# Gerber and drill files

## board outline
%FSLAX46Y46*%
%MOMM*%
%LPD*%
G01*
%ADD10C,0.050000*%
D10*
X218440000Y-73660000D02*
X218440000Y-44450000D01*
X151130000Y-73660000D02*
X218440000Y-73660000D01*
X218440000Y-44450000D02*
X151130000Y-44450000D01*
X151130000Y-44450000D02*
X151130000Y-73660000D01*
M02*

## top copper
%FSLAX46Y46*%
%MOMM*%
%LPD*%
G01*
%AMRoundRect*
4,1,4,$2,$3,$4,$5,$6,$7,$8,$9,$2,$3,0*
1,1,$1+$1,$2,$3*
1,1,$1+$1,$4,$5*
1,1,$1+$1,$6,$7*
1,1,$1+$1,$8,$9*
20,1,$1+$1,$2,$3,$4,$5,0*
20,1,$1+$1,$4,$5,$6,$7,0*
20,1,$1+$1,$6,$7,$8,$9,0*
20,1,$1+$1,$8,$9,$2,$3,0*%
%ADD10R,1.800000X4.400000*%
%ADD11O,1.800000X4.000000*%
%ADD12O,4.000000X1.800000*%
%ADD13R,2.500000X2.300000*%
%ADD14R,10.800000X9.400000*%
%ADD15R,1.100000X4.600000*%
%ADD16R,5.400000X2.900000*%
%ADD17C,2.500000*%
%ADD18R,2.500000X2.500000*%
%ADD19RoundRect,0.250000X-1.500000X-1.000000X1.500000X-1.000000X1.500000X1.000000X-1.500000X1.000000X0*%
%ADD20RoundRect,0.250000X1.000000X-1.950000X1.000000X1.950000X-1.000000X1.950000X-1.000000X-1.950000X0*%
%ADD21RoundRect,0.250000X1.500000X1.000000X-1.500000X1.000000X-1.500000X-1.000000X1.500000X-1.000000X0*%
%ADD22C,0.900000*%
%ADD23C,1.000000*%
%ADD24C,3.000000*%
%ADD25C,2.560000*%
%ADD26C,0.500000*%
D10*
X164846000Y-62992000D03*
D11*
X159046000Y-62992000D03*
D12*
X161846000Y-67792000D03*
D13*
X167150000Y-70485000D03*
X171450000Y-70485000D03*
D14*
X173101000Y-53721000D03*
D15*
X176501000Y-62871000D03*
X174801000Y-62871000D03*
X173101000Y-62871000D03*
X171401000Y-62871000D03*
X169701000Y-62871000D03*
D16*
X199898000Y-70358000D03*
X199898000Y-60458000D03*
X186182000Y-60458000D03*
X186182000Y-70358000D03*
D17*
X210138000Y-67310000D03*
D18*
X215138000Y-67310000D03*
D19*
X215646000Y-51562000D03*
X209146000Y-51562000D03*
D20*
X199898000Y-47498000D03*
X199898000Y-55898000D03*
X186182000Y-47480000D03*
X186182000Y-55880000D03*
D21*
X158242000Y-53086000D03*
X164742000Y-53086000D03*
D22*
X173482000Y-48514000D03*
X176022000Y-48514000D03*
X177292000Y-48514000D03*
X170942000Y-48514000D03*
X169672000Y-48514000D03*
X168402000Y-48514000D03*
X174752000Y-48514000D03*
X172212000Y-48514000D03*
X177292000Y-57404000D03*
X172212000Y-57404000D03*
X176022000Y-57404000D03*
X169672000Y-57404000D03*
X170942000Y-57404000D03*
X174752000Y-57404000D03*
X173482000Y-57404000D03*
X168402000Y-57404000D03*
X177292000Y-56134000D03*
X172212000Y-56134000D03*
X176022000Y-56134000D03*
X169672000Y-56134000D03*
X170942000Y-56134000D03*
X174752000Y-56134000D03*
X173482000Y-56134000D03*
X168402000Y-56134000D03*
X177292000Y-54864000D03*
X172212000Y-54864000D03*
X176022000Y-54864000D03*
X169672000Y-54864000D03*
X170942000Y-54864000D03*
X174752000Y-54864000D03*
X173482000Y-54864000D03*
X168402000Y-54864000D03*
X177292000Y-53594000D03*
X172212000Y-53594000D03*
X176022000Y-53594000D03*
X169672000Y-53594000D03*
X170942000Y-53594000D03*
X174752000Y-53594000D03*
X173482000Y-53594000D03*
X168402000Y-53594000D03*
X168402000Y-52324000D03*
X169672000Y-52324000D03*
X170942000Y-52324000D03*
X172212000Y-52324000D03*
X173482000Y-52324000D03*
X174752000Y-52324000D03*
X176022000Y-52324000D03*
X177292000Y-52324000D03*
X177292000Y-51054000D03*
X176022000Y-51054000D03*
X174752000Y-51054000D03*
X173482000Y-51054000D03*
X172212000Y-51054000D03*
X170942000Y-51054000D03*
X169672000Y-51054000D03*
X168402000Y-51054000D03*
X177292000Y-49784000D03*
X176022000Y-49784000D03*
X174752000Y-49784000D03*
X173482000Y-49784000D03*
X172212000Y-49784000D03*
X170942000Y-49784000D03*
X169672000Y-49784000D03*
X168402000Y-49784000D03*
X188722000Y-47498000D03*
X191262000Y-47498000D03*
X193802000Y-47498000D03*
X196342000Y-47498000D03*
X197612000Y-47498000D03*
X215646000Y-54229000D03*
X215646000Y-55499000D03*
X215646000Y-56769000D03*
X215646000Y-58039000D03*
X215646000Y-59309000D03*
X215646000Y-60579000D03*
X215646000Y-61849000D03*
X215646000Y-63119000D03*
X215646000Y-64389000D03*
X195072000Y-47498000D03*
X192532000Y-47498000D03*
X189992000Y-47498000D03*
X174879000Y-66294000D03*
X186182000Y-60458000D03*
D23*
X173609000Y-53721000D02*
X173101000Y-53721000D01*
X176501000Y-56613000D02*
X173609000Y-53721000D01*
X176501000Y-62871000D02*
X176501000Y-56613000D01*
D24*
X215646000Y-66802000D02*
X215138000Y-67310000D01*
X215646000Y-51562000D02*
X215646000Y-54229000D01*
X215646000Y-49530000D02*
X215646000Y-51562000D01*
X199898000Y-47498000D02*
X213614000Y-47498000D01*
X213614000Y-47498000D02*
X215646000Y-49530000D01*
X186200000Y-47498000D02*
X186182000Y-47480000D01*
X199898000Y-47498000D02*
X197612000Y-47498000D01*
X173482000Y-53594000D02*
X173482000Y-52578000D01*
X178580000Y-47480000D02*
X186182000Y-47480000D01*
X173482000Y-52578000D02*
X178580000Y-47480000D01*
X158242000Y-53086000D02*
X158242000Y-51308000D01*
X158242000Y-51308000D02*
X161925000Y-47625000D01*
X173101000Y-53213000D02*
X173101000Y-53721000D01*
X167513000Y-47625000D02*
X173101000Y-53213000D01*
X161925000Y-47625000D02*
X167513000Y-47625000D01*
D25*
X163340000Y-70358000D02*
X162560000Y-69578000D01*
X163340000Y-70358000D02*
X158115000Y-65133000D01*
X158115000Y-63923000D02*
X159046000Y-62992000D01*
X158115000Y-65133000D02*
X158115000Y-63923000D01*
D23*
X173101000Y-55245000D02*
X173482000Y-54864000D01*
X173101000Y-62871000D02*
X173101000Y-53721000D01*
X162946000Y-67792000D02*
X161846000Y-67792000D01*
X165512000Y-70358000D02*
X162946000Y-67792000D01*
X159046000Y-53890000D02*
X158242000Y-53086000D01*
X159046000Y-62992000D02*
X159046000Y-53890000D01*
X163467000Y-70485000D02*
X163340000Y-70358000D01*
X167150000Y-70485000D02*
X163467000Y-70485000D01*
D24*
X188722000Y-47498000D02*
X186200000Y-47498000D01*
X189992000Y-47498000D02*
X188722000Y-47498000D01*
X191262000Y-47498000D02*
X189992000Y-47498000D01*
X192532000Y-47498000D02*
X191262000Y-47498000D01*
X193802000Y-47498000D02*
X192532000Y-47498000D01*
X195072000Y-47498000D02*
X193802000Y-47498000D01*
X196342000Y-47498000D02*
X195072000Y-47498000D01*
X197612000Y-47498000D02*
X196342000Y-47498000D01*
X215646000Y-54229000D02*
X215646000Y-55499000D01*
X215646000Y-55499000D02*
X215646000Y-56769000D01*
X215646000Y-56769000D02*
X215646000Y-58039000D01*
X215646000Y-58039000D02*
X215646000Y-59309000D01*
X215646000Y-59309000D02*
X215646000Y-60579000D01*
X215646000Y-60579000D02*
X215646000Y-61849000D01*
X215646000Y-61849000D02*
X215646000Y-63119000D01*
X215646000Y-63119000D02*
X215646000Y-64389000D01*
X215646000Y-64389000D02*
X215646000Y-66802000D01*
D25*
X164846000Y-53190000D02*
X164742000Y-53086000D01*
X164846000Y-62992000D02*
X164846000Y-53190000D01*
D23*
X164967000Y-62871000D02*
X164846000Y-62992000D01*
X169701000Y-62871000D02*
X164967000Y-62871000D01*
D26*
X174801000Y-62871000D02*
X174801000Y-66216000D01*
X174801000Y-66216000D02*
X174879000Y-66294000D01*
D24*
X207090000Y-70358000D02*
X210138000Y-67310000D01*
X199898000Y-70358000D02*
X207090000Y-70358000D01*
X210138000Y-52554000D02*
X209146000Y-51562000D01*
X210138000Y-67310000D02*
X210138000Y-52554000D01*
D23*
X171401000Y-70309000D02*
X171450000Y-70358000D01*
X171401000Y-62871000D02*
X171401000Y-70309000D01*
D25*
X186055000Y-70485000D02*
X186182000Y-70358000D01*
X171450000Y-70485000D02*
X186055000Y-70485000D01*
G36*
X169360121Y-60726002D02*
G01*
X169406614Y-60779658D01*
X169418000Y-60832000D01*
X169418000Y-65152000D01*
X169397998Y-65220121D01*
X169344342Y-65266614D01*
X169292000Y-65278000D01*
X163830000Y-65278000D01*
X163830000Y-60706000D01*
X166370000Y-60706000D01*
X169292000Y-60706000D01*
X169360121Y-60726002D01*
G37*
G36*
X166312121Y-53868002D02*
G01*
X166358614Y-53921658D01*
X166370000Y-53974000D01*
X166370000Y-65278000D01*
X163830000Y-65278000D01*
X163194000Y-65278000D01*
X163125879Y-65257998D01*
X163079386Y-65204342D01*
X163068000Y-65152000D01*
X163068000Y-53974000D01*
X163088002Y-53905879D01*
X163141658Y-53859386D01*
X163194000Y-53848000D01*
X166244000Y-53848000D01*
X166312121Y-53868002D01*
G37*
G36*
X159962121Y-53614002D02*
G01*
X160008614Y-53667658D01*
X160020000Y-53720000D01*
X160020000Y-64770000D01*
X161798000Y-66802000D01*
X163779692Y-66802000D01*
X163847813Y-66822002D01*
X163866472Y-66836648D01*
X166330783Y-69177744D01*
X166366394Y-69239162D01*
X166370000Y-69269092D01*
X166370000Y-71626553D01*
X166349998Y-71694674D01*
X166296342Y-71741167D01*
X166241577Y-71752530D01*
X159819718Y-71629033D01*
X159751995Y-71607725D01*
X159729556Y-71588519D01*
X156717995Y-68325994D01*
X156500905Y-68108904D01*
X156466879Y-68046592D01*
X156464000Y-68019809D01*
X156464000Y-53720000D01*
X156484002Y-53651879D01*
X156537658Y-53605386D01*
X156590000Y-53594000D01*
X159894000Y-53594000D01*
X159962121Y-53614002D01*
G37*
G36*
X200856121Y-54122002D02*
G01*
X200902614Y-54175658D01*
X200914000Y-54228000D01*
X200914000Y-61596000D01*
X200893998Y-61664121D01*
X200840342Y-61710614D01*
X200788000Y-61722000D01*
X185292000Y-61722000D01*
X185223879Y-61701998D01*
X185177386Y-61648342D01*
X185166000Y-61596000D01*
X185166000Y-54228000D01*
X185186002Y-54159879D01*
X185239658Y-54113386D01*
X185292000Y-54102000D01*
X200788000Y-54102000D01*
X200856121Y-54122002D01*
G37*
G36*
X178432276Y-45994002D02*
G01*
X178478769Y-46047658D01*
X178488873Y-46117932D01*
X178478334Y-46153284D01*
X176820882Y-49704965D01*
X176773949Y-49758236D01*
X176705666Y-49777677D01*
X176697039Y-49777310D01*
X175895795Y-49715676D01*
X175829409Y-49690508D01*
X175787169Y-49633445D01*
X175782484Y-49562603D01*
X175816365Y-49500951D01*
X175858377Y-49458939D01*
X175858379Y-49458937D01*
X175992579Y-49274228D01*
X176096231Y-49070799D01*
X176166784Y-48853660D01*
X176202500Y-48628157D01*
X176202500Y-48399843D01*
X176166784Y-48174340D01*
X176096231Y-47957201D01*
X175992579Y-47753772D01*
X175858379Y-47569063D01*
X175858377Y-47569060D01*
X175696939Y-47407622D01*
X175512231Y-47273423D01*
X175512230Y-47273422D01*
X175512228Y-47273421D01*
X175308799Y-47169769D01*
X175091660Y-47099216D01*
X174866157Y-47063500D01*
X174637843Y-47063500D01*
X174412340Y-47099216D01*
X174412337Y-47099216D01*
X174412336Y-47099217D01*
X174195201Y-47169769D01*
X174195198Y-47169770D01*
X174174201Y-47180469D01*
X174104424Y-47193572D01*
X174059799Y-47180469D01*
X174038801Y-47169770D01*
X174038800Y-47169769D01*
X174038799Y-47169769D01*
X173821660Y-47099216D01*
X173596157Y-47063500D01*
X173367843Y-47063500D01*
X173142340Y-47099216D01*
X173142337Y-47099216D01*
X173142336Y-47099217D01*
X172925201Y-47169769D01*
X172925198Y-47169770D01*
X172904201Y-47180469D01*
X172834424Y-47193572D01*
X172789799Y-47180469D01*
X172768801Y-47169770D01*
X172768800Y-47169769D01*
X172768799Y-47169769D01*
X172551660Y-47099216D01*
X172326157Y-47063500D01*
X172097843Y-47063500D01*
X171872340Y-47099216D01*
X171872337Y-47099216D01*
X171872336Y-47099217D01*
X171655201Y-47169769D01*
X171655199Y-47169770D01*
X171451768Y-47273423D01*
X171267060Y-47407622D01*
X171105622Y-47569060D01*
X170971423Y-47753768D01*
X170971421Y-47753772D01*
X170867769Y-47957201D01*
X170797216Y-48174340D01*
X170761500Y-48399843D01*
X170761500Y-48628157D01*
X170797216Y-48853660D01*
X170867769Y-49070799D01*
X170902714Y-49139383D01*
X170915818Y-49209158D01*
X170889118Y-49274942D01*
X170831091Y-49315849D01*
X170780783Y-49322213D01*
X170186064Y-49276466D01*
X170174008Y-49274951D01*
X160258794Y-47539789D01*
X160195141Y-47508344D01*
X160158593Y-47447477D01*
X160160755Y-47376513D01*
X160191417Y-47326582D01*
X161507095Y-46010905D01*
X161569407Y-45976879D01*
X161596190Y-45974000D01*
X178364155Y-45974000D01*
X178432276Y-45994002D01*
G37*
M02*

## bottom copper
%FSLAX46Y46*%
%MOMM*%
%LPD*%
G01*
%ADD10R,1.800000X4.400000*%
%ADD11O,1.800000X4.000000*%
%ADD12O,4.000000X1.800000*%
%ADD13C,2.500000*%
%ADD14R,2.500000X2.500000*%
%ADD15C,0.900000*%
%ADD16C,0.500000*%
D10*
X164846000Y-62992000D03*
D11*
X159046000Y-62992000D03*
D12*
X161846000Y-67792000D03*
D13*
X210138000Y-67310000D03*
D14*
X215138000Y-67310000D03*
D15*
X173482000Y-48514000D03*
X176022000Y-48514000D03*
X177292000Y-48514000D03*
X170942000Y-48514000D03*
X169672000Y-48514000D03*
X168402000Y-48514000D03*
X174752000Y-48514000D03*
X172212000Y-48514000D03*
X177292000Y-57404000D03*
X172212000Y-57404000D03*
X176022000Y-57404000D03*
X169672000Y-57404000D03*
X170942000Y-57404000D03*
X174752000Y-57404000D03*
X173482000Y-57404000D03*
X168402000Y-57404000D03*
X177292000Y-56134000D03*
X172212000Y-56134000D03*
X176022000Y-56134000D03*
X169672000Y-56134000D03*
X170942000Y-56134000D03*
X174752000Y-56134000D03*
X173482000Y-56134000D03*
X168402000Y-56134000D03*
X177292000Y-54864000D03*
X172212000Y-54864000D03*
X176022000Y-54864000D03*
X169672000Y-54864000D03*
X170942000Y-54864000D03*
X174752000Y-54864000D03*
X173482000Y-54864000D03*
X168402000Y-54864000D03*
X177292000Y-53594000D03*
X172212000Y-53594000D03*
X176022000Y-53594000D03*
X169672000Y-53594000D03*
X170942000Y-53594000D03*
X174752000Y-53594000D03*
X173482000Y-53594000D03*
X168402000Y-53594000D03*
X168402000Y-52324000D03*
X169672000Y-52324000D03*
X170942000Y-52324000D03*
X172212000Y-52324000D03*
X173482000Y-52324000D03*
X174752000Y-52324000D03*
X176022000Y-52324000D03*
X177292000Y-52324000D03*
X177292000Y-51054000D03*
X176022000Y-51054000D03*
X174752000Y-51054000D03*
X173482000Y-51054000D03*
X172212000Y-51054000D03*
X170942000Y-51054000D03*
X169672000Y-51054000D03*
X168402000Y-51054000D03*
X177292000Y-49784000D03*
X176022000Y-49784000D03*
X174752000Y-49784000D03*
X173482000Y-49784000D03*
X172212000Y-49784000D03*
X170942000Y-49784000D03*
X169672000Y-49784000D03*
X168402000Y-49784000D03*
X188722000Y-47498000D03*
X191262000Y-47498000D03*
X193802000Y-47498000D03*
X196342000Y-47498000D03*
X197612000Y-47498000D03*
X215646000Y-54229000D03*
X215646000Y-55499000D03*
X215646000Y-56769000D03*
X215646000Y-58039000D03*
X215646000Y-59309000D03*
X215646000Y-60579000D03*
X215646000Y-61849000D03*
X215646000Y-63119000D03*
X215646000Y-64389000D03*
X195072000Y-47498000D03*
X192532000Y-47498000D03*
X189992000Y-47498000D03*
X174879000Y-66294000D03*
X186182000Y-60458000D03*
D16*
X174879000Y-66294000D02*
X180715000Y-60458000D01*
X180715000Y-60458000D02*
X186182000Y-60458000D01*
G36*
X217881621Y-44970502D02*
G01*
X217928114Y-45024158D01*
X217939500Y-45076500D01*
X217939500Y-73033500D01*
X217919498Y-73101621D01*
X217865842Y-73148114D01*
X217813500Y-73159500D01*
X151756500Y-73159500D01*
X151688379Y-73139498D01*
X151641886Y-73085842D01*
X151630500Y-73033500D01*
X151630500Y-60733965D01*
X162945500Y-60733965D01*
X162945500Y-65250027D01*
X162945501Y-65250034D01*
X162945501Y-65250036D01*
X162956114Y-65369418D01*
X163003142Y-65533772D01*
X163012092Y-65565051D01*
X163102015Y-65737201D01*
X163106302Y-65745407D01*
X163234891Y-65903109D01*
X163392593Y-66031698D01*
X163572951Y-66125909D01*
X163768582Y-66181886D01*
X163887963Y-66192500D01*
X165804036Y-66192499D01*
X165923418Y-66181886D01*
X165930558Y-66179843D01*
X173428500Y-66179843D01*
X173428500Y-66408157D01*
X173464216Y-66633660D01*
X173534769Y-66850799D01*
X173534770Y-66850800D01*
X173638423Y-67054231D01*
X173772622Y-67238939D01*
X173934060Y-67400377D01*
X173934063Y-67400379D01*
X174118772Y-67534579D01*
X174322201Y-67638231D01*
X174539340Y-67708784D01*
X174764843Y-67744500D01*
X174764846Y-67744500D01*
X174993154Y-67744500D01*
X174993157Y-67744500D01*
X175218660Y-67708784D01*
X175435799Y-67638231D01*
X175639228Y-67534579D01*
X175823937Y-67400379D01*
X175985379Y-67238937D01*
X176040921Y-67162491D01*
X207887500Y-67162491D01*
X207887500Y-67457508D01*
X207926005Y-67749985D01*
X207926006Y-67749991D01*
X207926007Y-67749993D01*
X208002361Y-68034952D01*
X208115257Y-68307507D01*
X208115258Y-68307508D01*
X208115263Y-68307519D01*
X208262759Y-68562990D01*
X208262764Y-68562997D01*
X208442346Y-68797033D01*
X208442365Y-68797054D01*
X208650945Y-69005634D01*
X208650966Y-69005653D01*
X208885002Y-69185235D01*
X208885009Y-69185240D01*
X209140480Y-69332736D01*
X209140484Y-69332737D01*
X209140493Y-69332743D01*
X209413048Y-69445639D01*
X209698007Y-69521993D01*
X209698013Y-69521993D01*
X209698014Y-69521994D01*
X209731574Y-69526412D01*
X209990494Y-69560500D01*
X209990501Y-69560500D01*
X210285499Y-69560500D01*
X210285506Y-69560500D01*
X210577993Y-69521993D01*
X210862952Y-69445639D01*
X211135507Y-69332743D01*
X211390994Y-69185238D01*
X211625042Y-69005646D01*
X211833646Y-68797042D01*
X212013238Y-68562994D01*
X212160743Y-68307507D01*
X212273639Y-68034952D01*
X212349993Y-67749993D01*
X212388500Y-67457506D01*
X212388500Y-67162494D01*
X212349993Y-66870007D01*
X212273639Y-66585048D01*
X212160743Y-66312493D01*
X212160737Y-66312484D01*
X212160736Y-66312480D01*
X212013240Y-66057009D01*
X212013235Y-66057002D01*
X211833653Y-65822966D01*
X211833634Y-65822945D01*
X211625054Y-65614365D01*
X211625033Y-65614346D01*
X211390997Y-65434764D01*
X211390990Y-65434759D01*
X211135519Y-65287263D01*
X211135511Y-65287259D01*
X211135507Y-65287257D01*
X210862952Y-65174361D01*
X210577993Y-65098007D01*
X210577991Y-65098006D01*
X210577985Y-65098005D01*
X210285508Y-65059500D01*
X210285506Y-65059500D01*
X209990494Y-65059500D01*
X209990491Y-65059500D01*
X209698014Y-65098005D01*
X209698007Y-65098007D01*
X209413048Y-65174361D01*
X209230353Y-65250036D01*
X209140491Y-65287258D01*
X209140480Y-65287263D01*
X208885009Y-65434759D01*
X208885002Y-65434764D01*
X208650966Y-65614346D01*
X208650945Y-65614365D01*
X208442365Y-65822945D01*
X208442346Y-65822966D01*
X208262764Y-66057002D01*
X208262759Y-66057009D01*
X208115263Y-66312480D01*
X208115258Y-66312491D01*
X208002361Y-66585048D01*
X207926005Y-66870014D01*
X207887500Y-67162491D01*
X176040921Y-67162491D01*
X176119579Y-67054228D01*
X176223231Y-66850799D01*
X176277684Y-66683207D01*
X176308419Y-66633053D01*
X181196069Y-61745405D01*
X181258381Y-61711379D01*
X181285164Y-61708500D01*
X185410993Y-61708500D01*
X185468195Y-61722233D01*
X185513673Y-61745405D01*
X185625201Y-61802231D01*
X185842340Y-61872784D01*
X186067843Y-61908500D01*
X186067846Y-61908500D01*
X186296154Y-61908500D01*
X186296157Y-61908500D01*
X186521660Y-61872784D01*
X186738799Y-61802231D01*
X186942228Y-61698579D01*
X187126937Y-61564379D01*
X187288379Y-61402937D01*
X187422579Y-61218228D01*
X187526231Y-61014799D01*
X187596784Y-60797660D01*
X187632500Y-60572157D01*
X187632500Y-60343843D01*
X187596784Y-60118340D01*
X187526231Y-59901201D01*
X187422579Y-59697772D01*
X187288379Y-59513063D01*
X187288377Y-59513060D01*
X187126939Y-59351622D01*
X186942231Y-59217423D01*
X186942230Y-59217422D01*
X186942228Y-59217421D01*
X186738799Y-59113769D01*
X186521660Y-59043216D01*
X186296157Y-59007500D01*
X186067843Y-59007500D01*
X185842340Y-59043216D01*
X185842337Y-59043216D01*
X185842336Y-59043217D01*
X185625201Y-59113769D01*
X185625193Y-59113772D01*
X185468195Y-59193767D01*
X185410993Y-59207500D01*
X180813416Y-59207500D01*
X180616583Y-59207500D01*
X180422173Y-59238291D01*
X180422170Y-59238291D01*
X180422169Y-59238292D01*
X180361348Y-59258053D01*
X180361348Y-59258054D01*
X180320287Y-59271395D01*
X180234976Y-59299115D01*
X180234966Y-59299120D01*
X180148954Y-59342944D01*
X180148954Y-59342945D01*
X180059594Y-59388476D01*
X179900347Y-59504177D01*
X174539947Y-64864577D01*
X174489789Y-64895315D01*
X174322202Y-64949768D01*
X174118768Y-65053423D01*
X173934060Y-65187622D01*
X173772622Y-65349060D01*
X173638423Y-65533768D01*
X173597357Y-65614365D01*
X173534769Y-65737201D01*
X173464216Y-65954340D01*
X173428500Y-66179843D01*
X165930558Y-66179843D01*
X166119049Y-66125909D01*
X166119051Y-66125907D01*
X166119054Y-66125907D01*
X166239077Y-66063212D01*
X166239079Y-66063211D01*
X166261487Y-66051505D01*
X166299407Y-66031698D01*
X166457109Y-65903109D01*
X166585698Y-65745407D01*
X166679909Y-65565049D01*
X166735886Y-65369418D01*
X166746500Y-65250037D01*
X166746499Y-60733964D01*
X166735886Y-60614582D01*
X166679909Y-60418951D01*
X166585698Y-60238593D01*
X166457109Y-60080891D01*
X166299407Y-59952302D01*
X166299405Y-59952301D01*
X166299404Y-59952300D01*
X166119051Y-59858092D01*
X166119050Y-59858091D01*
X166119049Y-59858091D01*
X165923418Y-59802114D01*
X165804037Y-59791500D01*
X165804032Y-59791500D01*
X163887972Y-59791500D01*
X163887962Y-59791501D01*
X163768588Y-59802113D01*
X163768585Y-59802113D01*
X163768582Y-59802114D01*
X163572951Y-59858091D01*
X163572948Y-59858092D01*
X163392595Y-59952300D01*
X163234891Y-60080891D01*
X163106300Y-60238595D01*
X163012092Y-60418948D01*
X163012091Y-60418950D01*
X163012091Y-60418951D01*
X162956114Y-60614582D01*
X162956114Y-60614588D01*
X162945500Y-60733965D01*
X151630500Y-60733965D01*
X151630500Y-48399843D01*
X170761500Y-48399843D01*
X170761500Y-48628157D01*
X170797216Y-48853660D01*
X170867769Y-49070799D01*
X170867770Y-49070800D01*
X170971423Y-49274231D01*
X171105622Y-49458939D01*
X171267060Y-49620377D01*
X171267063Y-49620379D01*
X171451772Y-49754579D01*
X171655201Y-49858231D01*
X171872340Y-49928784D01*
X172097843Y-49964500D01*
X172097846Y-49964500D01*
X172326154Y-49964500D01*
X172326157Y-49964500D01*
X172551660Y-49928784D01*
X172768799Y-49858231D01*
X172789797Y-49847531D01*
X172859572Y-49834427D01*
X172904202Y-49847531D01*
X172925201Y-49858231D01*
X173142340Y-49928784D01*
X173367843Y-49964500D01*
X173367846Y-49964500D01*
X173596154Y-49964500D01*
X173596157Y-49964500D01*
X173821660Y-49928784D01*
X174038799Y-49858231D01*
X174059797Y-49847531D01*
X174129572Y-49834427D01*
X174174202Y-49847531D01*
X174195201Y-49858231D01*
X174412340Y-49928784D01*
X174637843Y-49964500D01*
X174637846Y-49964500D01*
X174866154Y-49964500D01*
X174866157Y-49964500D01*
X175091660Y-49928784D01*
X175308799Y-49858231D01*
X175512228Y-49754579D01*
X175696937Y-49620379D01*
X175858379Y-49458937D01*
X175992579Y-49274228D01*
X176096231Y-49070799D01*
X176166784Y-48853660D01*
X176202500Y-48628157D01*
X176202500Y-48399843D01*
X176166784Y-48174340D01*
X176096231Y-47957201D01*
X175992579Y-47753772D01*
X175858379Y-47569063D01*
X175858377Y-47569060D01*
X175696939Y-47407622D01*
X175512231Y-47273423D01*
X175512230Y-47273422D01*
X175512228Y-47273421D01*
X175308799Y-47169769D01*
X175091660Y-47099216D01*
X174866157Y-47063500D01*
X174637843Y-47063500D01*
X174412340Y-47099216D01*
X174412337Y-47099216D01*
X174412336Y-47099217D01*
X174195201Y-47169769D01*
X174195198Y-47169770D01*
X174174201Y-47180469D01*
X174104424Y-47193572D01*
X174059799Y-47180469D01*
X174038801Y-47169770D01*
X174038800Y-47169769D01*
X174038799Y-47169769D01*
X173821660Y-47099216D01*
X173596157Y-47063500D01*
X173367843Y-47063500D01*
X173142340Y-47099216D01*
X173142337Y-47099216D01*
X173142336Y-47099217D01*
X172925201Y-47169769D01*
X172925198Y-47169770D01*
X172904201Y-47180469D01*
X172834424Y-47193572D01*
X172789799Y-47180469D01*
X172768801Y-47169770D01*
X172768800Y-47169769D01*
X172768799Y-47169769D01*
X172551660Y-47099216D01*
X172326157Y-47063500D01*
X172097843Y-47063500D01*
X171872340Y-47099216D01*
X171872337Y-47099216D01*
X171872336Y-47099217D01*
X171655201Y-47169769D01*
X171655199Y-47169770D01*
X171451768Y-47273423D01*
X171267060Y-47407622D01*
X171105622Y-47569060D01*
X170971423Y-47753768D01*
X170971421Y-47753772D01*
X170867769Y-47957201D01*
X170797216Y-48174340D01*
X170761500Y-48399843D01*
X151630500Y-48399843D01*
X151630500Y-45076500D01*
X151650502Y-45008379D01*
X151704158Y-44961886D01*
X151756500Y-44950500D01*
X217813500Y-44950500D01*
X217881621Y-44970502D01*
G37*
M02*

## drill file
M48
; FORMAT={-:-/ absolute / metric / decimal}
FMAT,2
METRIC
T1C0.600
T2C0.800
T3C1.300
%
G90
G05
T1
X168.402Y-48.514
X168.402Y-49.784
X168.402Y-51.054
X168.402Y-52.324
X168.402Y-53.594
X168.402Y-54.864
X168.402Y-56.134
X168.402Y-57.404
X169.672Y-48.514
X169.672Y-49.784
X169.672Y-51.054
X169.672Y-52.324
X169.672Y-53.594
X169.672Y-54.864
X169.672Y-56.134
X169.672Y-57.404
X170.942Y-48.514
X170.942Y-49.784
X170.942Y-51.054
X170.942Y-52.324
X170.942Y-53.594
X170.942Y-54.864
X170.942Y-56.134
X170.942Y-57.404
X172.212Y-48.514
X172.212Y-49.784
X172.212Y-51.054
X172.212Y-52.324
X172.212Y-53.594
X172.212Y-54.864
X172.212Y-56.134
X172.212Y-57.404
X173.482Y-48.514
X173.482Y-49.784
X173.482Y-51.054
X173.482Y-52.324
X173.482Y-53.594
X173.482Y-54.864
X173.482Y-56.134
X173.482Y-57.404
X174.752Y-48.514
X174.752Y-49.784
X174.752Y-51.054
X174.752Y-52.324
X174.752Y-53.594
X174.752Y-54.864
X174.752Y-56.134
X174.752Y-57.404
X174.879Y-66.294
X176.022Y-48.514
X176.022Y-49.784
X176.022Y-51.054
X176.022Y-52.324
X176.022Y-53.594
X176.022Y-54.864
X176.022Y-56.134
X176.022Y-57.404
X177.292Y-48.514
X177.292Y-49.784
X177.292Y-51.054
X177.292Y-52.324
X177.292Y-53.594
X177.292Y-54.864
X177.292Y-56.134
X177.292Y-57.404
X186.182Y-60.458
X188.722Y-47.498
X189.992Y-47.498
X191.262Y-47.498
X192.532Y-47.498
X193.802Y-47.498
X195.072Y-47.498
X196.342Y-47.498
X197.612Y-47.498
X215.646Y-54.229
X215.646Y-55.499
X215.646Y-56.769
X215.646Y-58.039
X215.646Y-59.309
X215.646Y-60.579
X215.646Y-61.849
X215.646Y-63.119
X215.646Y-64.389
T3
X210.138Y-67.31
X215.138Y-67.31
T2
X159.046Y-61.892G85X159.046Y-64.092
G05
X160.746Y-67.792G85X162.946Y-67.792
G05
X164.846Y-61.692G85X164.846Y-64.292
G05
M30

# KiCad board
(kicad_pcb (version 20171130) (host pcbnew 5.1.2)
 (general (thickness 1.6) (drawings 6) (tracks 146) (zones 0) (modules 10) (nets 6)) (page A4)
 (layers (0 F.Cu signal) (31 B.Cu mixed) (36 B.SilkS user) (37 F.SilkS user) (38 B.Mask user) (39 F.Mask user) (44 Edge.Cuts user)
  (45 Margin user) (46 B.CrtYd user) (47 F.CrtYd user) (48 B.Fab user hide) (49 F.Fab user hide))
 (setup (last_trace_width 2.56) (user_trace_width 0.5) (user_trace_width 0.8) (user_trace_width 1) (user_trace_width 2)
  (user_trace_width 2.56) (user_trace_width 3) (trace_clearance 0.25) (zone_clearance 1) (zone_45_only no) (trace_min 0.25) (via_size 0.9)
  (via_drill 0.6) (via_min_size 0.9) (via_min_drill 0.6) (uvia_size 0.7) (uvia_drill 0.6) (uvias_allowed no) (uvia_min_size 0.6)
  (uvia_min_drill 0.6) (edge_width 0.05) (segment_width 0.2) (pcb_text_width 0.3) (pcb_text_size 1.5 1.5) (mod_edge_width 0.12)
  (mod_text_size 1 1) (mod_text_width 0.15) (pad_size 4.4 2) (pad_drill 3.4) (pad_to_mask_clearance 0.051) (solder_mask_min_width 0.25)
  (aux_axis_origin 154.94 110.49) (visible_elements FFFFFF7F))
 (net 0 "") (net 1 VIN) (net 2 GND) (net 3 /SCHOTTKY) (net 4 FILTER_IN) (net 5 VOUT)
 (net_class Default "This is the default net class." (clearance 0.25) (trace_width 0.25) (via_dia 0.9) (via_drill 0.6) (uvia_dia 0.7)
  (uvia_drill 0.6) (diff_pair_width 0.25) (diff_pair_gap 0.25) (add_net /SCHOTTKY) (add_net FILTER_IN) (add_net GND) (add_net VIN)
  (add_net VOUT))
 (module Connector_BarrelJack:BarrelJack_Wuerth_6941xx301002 (layer F.Cu) (at 164.846 62.992 270)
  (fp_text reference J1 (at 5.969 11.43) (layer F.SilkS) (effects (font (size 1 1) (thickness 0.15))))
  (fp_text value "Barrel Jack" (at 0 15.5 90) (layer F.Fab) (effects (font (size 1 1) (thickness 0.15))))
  (pad 1 thru_hole rect (at 0 0 270) (size 4.4 1.8) (drill oval 3.4 0.8) (layers *.Cu *.Mask) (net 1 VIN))
  (pad 2 thru_hole oval (at 0 5.8 270) (size 4 1.8) (drill oval 3 0.8) (layers *.Cu *.Mask) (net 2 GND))
  (pad 3 thru_hole oval (at 4.8 3) (size 4 1.8) (drill oval 3 0.8) (layers *.Cu *.Mask) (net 2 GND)))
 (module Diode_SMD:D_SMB (layer F.Cu) (at 169.3 70.485 180)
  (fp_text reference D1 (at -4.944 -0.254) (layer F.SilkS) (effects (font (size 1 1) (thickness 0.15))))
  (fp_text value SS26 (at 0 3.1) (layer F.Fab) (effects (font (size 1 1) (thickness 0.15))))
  (pad 2 smd rect (at 2.15 0 180) (size 2.5 2.3) (layers F.Cu F.Paste F.Mask) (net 2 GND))
  (pad 1 smd rect (at -2.15 0 180) (size 2.5 2.3) (layers F.Cu F.Paste F.Mask) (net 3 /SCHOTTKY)))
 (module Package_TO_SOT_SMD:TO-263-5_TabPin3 (layer F.Cu) (at 173.101 57.096 90)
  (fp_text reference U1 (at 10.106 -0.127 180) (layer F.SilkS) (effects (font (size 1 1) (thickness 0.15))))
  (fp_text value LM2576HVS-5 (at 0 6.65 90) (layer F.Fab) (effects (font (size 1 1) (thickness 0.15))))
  (pad "" smd rect (at 0.95 2.775 90) (size 4.55 5.25) (layers F.Paste))
  (pad "" smd rect (at 5.8 -2.775 90) (size 4.55 5.25) (layers F.Paste))
  (pad "" smd rect (at 0.95 -2.775 90) (size 4.55 5.25) (layers F.Paste))
  (pad "" smd rect (at 5.8 2.775 90) (size 4.55 5.25) (layers F.Paste))
  (pad 3 smd rect (at 3.375 0 90) (size 9.4 10.8) (layers F.Cu F.Mask) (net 2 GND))
  (pad 5 smd rect (at -5.775 3.4 90) (size 4.6 1.1) (layers F.Cu F.Paste F.Mask) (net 2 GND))
  (pad 4 smd rect (at -5.775 1.7 90) (size 4.6 1.1) (layers F.Cu F.Paste F.Mask) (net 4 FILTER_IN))
  (pad 3 smd rect (at -5.775 0 90) (size 4.6 1.1) (layers F.Cu F.Paste F.Mask) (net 2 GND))
  (pad 2 smd rect (at -5.775 -1.7 90) (size 4.6 1.1) (layers F.Cu F.Paste F.Mask) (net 3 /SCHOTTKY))
  (pad 1 smd rect (at -5.775 -3.4 90) (size 4.6 1.1) (layers F.Cu F.Paste F.Mask) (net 1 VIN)))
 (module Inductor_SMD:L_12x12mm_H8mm (layer F.Cu) (at 199.898 65.408 270)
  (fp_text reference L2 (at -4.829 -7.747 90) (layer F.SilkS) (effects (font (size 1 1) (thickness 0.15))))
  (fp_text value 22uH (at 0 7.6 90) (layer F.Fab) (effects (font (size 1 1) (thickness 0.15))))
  (pad 2 smd rect (at 4.95 0 270) (size 2.9 5.4) (layers F.Cu F.Paste F.Mask) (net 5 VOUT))
  (pad 1 smd rect (at -4.95 0 270) (size 2.9 5.4) (layers F.Cu F.Paste F.Mask) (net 4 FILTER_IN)))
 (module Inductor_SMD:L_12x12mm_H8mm (layer F.Cu) (at 186.182 65.408 90)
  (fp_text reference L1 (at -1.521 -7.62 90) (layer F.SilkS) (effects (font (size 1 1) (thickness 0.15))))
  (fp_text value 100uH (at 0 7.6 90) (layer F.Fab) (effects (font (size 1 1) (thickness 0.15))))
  (pad 2 smd rect (at 4.95 0 90) (size 2.9 5.4) (layers F.Cu F.Paste F.Mask) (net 4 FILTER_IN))
  (pad 1 smd rect (at -4.95 0 90) (size 2.9 5.4) (layers F.Cu F.Paste F.Mask) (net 3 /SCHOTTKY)))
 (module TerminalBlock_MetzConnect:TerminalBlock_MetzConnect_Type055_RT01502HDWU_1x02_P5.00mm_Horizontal (layer F.Cu) (at 215.138 67.31 180)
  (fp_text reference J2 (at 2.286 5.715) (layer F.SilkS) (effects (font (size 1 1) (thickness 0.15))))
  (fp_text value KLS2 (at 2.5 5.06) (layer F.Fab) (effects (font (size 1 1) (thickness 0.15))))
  (pad 2 thru_hole circle (at 5 0 180) (size 2.5 2.5) (drill 1.3) (layers *.Cu *.Mask) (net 5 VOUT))
  (pad 1 thru_hole rect (at 0 0 180) (size 2.5 2.5) (drill 1.3) (layers *.Cu *.Mask) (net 2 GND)))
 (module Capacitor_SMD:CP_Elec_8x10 (layer F.Cu) (at 212.396 51.562)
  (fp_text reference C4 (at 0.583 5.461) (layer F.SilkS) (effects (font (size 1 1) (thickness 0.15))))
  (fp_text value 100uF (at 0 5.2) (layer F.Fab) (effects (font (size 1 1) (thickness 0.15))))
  (pad 2 smd roundrect (at 3.25 0) (size 3.5 2.5) (layers F.Cu F.Paste F.Mask) (roundrect_rratio 0.1) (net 2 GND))
  (pad 1 smd roundrect (at -3.25 0) (size 3.5 2.5) (layers F.Cu F.Paste F.Mask) (roundrect_rratio 0.1) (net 5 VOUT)))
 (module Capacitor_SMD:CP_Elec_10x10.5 (layer F.Cu) (at 199.898 51.698 90)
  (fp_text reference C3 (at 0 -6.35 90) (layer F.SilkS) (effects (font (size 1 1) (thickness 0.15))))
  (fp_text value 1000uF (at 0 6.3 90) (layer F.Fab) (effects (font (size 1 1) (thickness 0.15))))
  (pad 2 smd roundrect (at 4.2 0 90) (size 4.4 2.5) (layers F.Cu F.Paste F.Mask) (roundrect_rratio 0.1) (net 2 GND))
  (pad 1 smd roundrect (at -4.2 0 90) (size 4.4 2.5) (layers F.Cu F.Paste F.Mask) (roundrect_rratio 0.1) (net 4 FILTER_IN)))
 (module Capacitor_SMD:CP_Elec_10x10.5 (layer F.Cu) (at 186.182 51.68 90)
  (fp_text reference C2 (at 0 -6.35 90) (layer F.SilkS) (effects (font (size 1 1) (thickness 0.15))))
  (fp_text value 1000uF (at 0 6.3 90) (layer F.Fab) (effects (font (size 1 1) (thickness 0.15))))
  (pad 2 smd roundrect (at 4.2 0 90) (size 4.4 2.5) (layers F.Cu F.Paste F.Mask) (roundrect_rratio 0.1) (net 2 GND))
  (pad 1 smd roundrect (at -4.2 0 90) (size 4.4 2.5) (layers F.Cu F.Paste F.Mask) (roundrect_rratio 0.1) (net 4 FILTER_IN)))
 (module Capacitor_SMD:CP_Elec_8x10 (layer F.Cu) (at 161.492 53.086 180)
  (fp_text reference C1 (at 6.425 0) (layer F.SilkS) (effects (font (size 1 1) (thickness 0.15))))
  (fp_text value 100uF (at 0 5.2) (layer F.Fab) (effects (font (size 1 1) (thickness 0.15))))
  (pad 2 smd roundrect (at 3.25 0 180) (size 3.5 2.5) (layers F.Cu F.Paste F.Mask) (roundrect_rratio 0.1) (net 2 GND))
  (pad 1 smd roundrect (at -3.25 0 180) (size 3.5 2.5) (layers F.Cu F.Paste F.Mask) (roundrect_rratio 0.1) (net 1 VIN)))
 (gr_line (start 218.44 73.66) (end 218.44 44.45) (layer Edge.Cuts) (width 0.05))
 (gr_line (start 151.13 73.66) (end 218.44 73.66) (layer Edge.Cuts) (width 0.05))
 (gr_line (start 218.44 44.45) (end 151.13 44.45) (layer Edge.Cuts) (width 0.05))
 (gr_line (start 151.13 44.45) (end 151.13 73.66) (layer Edge.Cuts) (width 0.05))
 (via (at 173.482 48.514) (size 0.9) (drill 0.6) (layers F.Cu B.Cu) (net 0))
 (via (at 176.022 48.514) (size 0.9) (drill 0.6) (layers F.Cu B.Cu) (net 2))
 (via (at 177.292 48.514) (size 0.9) (drill 0.6) (layers F.Cu B.Cu) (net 2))
 (via (at 170.942 48.514) (size 0.9) (drill 0.6) (layers F.Cu B.Cu) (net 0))
 (via (at 169.672 48.514) (size 0.9) (drill 0.6) (layers F.Cu B.Cu) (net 2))
 (via (at 168.402 48.514) (size 0.9) (drill 0.6) (layers F.Cu B.Cu) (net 2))
 (via (at 174.752 48.514) (size 0.9) (drill 0.6) (layers F.Cu B.Cu) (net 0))
 (via (at 172.212 48.514) (size 0.9) (drill 0.6) (layers F.Cu B.Cu) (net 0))
 (via (at 177.292 57.404) (size 0.9) (drill 0.6) (layers F.Cu B.Cu) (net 2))
 (via (at 172.212 57.404) (size 0.9) (drill 0.6) (layers F.Cu B.Cu) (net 2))
 (via (at 176.022 57.404) (size 0.9) (drill 0.6) (layers F.Cu B.Cu) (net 2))
 (via (at 169.672 57.404) (size 0.9) (drill 0.6) (layers F.Cu B.Cu) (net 2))
 (via (at 170.942 57.404) (size 0.9) (drill 0.6) (layers F.Cu B.Cu) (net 2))
 (via (at 174.752 57.404) (size 0.9) (drill 0.6) (layers F.Cu B.Cu) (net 2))
 (via (at 173.482 57.404) (size 0.9) (drill 0.6) (layers F.Cu B.Cu) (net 2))
 (via (at 168.402 57.404) (size 0.9) (drill 0.6) (layers F.Cu B.Cu) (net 2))
 (via (at 177.292 56.134) (size 0.9) (drill 0.6) (layers F.Cu B.Cu) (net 2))
 (via (at 172.212 56.134) (size 0.9) (drill 0.6) (layers F.Cu B.Cu) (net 2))
 (via (at 176.022 56.134) (size 0.9) (drill 0.6) (layers F.Cu B.Cu) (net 2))
 (via (at 169.672 56.134) (size 0.9) (drill 0.6) (layers F.Cu B.Cu) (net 2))
 (via (at 170.942 56.134) (size 0.9) (drill 0.6) (layers F.Cu B.Cu) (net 2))
 (via (at 174.752 56.134) (size 0.9) (drill 0.6) (layers F.Cu B.Cu) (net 2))
 (via (at 173.482 56.134) (size 0.9) (drill 0.6) (layers F.Cu B.Cu) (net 2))
 (via (at 168.402 56.134) (size 0.9) (drill 0.6) (layers F.Cu B.Cu) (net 2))
 (via (at 177.292 54.864) (size 0.9) (drill 0.6) (layers F.Cu B.Cu) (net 2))
 (via (at 172.212 54.864) (size 0.9) (drill 0.6) (layers F.Cu B.Cu) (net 2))
 (via (at 176.022 54.864) (size 0.9) (drill 0.6) (layers F.Cu B.Cu) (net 2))
 (via (at 169.672 54.864) (size 0.9) (drill 0.6) (layers F.Cu B.Cu) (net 2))
 (via (at 170.942 54.864) (size 0.9) (drill 0.6) (layers F.Cu B.Cu) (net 2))
 (via (at 174.752 54.864) (size 0.9) (drill 0.6) (layers F.Cu B.Cu) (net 2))
 (via (at 173.482 54.864) (size 0.9) (drill 0.6) (layers F.Cu B.Cu) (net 2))
 (via (at 168.402 54.864) (size 0.9) (drill 0.6) (layers F.Cu B.Cu) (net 2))
 (via (at 177.292 53.594) (size 0.9) (drill 0.6) (layers F.Cu B.Cu) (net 2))
 (via (at 172.212 53.594) (size 0.9) (drill 0.6) (layers F.Cu B.Cu) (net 2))
 (via (at 176.022 53.594) (size 0.9) (drill 0.6) (layers F.Cu B.Cu) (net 2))
 (via (at 169.672 53.594) (size 0.9) (drill 0.6) (layers F.Cu B.Cu) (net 2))
 (via (at 170.942 53.594) (size 0.9) (drill 0.6) (layers F.Cu B.Cu) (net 2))
 (via (at 174.752 53.594) (size 0.9) (drill 0.6) (layers F.Cu B.Cu) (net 2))
 (via (at 173.482 53.594) (size 0.9) (drill 0.6) (layers F.Cu B.Cu) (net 2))
 (via (at 168.402 53.594) (size 0.9) (drill 0.6) (layers F.Cu B.Cu) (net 2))
 (via (at 168.402 52.324) (size 0.9) (drill 0.6) (layers F.Cu B.Cu) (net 2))
 (via (at 169.672 52.324) (size 0.9) (drill 0.6) (layers F.Cu B.Cu) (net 2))
 (via (at 170.942 52.324) (size 0.9) (drill 0.6) (layers F.Cu B.Cu) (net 2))
 (via (at 172.212 52.324) (size 0.9) (drill 0.6) (layers F.Cu B.Cu) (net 2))
 (via (at 173.482 52.324) (size 0.9) (drill 0.6) (layers F.Cu B.Cu) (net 2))
 (via (at 174.752 52.324) (size 0.9) (drill 0.6) (layers F.Cu B.Cu) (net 2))
 (via (at 176.022 52.324) (size 0.9) (drill 0.6) (layers F.Cu B.Cu) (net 2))
 (via (at 177.292 52.324) (size 0.9) (drill 0.6) (layers F.Cu B.Cu) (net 2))
 (via (at 177.292 51.054) (size 0.9) (drill 0.6) (layers F.Cu B.Cu) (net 2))
 (via (at 176.022 51.054) (size 0.9) (drill 0.6) (layers F.Cu B.Cu) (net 2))
 (via (at 174.752 51.054) (size 0.9) (drill 0.6) (layers F.Cu B.Cu) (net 2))
 (via (at 173.482 51.054) (size 0.9) (drill 0.6) (layers F.Cu B.Cu) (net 2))
 (via (at 172.212 51.054) (size 0.9) (drill 0.6) (layers F.Cu B.Cu) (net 2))
 (via (at 170.942 51.054) (size 0.9) (drill 0.6) (layers F.Cu B.Cu) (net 2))
 (via (at 169.672 51.054) (size 0.9) (drill 0.6) (layers F.Cu B.Cu) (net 2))
 (via (at 168.402 51.054) (size 0.9) (drill 0.6) (layers F.Cu B.Cu) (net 2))
 (via (at 177.292 49.784) (size 0.9) (drill 0.6) (layers F.Cu B.Cu) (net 2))
 (via (at 176.022 49.784) (size 0.9) (drill 0.6) (layers F.Cu B.Cu) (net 2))
 (via (at 174.752 49.784) (size 0.9) (drill 0.6) (layers F.Cu B.Cu) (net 2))
 (via (at 173.482 49.784) (size 0.9) (drill 0.6) (layers F.Cu B.Cu) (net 2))
 (via (at 172.212 49.784) (size 0.9) (drill 0.6) (layers F.Cu B.Cu) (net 2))
 (via (at 170.942 49.784) (size 0.9) (drill 0.6) (layers F.Cu B.Cu) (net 2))
 (via (at 169.672 49.784) (size 0.9) (drill 0.6) (layers F.Cu B.Cu) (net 2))
 (via (at 168.402 49.784) (size 0.9) (drill 0.6) (layers F.Cu B.Cu) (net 2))
 (segment (start 173.609 53.721) (end 173.101 53.721) (width 1) (layer F.Cu) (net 2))
 (segment (start 176.501 56.613) (end 173.609 53.721) (width 1) (layer F.Cu) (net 2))
 (segment (start 176.501 62.871) (end 176.501 56.613) (width 1) (layer F.Cu) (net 2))
 (segment (start 215.646 66.802) (end 215.138 67.31) (width 3) (layer F.Cu) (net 2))
 (segment (start 215.646 51.562) (end 215.646 54.229) (width 3) (layer F.Cu) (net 2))
 (segment (start 215.646 49.53) (end 215.646 51.562) (width 3) (layer F.Cu) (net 2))
 (segment (start 199.898 47.498) (end 213.614 47.498) (width 3) (layer F.Cu) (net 2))
 (segment (start 213.614 47.498) (end 215.646 49.53) (width 3) (layer F.Cu) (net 2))
 (segment (start 186.2 47.498) (end 186.182 47.48) (width 3) (layer F.Cu) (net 2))
 (segment (start 199.898 47.498) (end 197.612 47.498) (width 3) (layer F.Cu) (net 2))
 (segment (start 173.482 53.594) (end 173.482 52.578) (width 3) (layer F.Cu) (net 2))
 (segment (start 178.58 47.48) (end 186.182 47.48) (width 3) (layer F.Cu) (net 2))
 (segment (start 173.482 52.578) (end 178.58 47.48) (width 3) (layer F.Cu) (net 2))
 (segment (start 158.242 53.086) (end 158.242 51.308) (width 3) (layer F.Cu) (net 2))
 (segment (start 158.242 51.308) (end 161.925 47.625) (width 3) (layer F.Cu) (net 2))
 (segment (start 173.101 53.213) (end 173.101 53.721) (width 3) (layer F.Cu) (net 2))
 (segment (start 167.513 47.625) (end 173.101 53.213) (width 3) (layer F.Cu) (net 2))
 (segment (start 161.925 47.625) (end 167.513 47.625) (width 3) (layer F.Cu) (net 2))
 (segment (start 163.34 70.358) (end 162.56 69.578) (width 2.56) (layer F.Cu) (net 2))
 (segment (start 163.34 70.358) (end 158.115 65.133) (width 2.56) (layer F.Cu) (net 2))
 (segment (start 158.115 63.923) (end 159.046 62.992) (width 2.56) (layer F.Cu) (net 2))
 (segment (start 158.115 65.133) (end 158.115 63.923) (width 2.56) (layer F.Cu) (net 2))
 (segment (start 173.101 55.245) (end 173.482 54.864) (width 1) (layer F.Cu) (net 2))
 (segment (start 173.101 62.871) (end 173.101 53.721) (width 1) (layer F.Cu) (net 2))
 (segment (start 162.946 67.792) (end 161.846 67.792) (width 1) (layer F.Cu) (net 2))
 (segment (start 165.512 70.358) (end 162.946 67.792) (width 1) (layer F.Cu) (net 2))
 (segment (start 159.046 53.89) (end 158.242 53.086) (width 1) (layer F.Cu) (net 2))
 (segment (start 159.046 62.992) (end 159.046 53.89) (width 1) (layer F.Cu) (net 2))
 (segment (start 163.467 70.485) (end 163.34 70.358) (width 1) (layer F.Cu) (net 2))
 (segment (start 167.15 70.485) (end 163.467 70.485) (width 1) (layer F.Cu) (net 2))
 (segment (start 188.722 47.498) (end 186.2 47.498) (width 3) (layer F.Cu) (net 2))
 (via (at 188.722 47.498) (size 0.9) (drill 0.6) (layers F.Cu B.Cu) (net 2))
 (segment (start 189.992 47.498) (end 188.722 47.498) (width 3) (layer F.Cu) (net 2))
 (segment (start 191.262 47.498) (end 189.992 47.498) (width 3) (layer F.Cu) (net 2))
 (via (at 191.262 47.498) (size 0.9) (drill 0.6) (layers F.Cu B.Cu) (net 2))
 (segment (start 192.532 47.498) (end 191.262 47.498) (width 3) (layer F.Cu) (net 2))
 (segment (start 193.802 47.498) (end 192.532 47.498) (width 3) (layer F.Cu) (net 2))
 (via (at 193.802 47.498) (size 0.9) (drill 0.6) (layers F.Cu B.Cu) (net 2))
 (segment (start 195.072 47.498) (end 193.802 47.498) (width 3) (layer F.Cu) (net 2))
 (segment (start 196.342 47.498) (end 195.072 47.498) (width 3) (layer F.Cu) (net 2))
 (via (at 196.342 47.498) (size 0.9) (drill 0.6) (layers F.Cu B.Cu) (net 2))
 (segment (start 197.612 47.498) (end 196.342 47.498) (width 3) (layer F.Cu) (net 2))
 (via (at 197.612 47.498) (size 0.9) (drill 0.6) (layers F.Cu B.Cu) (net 2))
 (segment (start 215.646 54.229) (end 215.646 55.499) (width 3) (layer F.Cu) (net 2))
 (via (at 215.646 54.229) (size 0.9) (drill 0.6) (layers F.Cu B.Cu) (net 2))
 (segment (start 215.646 55.499) (end 215.646 56.769) (width 3) (layer F.Cu) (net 2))
 (via (at 215.646 55.499) (size 0.9) (drill 0.6) (layers F.Cu B.Cu) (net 2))
 (segment (start 215.646 56.769) (end 215.646 58.039) (width 3) (layer F.Cu) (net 2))
 (via (at 215.646 56.769) (size 0.9) (drill 0.6) (layers F.Cu B.Cu) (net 2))
 (segment (start 215.646 58.039) (end 215.646 59.309) (width 3) (layer F.Cu) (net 2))
 (via (at 215.646 58.039) (size 0.9) (drill 0.6) (layers F.Cu B.Cu) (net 2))
 (segment (start 215.646 59.309) (end 215.646 60.579) (width 3) (layer F.Cu) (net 2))
 (via (at 215.646 59.309) (size 0.9) (drill 0.6) (layers F.Cu B.Cu) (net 2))
 (segment (start 215.646 60.579) (end 215.646 61.849) (width 3) (layer F.Cu) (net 2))
 (via (at 215.646 60.579) (size 0.9) (drill 0.6) (layers F.Cu B.Cu) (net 2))
 (segment (start 215.646 61.849) (end 215.646 63.119) (width 3) (layer F.Cu) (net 2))
 (via (at 215.646 61.849) (size 0.9) (drill 0.6) (layers F.Cu B.Cu) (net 2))
 (segment (start 215.646 63.119) (end 215.646 64.389) (width 3) (layer F.Cu) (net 2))
 (via (at 215.646 63.119) (size 0.9) (drill 0.6) (layers F.Cu B.Cu) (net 2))
 (segment (start 215.646 64.389) (end 215.646 66.802) (width 3) (layer F.Cu) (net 2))
 (via (at 215.646 64.389) (size 0.9) (drill 0.6) (layers F.Cu B.Cu) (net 2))
 (via (at 195.072 47.498) (size 0.9) (drill 0.6) (layers F.Cu B.Cu) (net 2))
 (via (at 192.532 47.498) (size 0.9) (drill 0.6) (layers F.Cu B.Cu) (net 2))
 (via (at 189.992 47.498) (size 0.9) (drill 0.6) (layers F.Cu B.Cu) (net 2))
 (segment (start 164.846 53.19) (end 164.742 53.086) (width 2.56) (layer F.Cu) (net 1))
 (segment (start 164.846 62.992) (end 164.846 53.19) (width 2.56) (layer F.Cu) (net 1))
 (segment (start 164.967 62.871) (end 164.846 62.992) (width 1) (layer F.Cu) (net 1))
 (segment (start 169.701 62.871) (end 164.967 62.871) (width 1) (layer F.Cu) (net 1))
 (via (at 174.879 66.294) (size 0.9) (drill 0.6) (layers F.Cu B.Cu) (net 4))
 (segment (start 174.801 62.871) (end 174.801 66.216) (width 0.5) (layer F.Cu) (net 4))
 (segment (start 174.801 66.216) (end 174.879 66.294) (width 0.5) (layer F.Cu) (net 4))
 (via (at 186.182 60.458) (size 0.9) (drill 0.6) (layers F.Cu B.Cu) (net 4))
 (segment (start 174.879 66.294) (end 180.715 60.458) (width 0.5) (layer B.Cu) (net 4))
 (segment (start 180.715 60.458) (end 186.182 60.458) (width 0.5) (layer B.Cu) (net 4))
 (segment (start 207.09 70.358) (end 210.138 67.31) (width 3) (layer F.Cu) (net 5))
 (segment (start 199.898 70.358) (end 207.09 70.358) (width 3) (layer F.Cu) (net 5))
 (segment (start 210.138 52.554) (end 209.146 51.562) (width 3) (layer F.Cu) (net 5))
 (segment (start 210.138 67.31) (end 210.138 52.554) (width 3) (layer F.Cu) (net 5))
 (segment (start 171.401 70.309) (end 171.45 70.358) (width 1) (layer F.Cu) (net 3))
 (segment (start 171.401 62.871) (end 171.401 70.309) (width 1) (layer F.Cu) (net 3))
 (segment (start 186.055 70.485) (end 186.182 70.358) (width 2.56) (layer F.Cu) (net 3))
 (segment (start 171.45 70.485) (end 186.055 70.485) (width 2.56) (layer F.Cu) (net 3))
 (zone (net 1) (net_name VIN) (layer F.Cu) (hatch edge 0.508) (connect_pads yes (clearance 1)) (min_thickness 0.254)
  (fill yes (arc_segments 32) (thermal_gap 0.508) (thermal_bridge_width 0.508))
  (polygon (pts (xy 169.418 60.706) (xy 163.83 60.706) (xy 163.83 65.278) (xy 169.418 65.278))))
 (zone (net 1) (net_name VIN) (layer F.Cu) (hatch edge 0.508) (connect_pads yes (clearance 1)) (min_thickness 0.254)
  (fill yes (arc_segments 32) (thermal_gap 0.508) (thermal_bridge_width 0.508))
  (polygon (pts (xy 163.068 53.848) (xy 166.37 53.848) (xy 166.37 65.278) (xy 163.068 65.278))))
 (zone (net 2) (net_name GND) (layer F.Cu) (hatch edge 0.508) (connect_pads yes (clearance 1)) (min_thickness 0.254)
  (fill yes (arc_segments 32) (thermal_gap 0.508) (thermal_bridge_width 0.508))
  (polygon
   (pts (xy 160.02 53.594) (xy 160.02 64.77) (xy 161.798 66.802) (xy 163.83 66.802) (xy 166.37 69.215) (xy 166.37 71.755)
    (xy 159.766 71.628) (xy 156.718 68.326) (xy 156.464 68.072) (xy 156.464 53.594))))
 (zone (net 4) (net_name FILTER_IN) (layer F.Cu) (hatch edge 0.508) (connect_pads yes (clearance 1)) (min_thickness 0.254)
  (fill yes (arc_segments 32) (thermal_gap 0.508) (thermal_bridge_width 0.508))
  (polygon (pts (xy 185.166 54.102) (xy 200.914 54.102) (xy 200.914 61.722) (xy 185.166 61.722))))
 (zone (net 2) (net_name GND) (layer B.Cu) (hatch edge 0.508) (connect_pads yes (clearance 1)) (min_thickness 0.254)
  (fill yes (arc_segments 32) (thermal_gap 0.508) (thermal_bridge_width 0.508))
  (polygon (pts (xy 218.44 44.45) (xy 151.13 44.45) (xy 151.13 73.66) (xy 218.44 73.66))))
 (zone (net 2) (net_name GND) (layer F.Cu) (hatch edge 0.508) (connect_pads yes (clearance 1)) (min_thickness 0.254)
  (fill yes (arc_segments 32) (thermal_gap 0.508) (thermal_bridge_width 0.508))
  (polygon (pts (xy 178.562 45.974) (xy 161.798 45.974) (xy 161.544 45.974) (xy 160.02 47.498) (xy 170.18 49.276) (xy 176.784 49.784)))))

